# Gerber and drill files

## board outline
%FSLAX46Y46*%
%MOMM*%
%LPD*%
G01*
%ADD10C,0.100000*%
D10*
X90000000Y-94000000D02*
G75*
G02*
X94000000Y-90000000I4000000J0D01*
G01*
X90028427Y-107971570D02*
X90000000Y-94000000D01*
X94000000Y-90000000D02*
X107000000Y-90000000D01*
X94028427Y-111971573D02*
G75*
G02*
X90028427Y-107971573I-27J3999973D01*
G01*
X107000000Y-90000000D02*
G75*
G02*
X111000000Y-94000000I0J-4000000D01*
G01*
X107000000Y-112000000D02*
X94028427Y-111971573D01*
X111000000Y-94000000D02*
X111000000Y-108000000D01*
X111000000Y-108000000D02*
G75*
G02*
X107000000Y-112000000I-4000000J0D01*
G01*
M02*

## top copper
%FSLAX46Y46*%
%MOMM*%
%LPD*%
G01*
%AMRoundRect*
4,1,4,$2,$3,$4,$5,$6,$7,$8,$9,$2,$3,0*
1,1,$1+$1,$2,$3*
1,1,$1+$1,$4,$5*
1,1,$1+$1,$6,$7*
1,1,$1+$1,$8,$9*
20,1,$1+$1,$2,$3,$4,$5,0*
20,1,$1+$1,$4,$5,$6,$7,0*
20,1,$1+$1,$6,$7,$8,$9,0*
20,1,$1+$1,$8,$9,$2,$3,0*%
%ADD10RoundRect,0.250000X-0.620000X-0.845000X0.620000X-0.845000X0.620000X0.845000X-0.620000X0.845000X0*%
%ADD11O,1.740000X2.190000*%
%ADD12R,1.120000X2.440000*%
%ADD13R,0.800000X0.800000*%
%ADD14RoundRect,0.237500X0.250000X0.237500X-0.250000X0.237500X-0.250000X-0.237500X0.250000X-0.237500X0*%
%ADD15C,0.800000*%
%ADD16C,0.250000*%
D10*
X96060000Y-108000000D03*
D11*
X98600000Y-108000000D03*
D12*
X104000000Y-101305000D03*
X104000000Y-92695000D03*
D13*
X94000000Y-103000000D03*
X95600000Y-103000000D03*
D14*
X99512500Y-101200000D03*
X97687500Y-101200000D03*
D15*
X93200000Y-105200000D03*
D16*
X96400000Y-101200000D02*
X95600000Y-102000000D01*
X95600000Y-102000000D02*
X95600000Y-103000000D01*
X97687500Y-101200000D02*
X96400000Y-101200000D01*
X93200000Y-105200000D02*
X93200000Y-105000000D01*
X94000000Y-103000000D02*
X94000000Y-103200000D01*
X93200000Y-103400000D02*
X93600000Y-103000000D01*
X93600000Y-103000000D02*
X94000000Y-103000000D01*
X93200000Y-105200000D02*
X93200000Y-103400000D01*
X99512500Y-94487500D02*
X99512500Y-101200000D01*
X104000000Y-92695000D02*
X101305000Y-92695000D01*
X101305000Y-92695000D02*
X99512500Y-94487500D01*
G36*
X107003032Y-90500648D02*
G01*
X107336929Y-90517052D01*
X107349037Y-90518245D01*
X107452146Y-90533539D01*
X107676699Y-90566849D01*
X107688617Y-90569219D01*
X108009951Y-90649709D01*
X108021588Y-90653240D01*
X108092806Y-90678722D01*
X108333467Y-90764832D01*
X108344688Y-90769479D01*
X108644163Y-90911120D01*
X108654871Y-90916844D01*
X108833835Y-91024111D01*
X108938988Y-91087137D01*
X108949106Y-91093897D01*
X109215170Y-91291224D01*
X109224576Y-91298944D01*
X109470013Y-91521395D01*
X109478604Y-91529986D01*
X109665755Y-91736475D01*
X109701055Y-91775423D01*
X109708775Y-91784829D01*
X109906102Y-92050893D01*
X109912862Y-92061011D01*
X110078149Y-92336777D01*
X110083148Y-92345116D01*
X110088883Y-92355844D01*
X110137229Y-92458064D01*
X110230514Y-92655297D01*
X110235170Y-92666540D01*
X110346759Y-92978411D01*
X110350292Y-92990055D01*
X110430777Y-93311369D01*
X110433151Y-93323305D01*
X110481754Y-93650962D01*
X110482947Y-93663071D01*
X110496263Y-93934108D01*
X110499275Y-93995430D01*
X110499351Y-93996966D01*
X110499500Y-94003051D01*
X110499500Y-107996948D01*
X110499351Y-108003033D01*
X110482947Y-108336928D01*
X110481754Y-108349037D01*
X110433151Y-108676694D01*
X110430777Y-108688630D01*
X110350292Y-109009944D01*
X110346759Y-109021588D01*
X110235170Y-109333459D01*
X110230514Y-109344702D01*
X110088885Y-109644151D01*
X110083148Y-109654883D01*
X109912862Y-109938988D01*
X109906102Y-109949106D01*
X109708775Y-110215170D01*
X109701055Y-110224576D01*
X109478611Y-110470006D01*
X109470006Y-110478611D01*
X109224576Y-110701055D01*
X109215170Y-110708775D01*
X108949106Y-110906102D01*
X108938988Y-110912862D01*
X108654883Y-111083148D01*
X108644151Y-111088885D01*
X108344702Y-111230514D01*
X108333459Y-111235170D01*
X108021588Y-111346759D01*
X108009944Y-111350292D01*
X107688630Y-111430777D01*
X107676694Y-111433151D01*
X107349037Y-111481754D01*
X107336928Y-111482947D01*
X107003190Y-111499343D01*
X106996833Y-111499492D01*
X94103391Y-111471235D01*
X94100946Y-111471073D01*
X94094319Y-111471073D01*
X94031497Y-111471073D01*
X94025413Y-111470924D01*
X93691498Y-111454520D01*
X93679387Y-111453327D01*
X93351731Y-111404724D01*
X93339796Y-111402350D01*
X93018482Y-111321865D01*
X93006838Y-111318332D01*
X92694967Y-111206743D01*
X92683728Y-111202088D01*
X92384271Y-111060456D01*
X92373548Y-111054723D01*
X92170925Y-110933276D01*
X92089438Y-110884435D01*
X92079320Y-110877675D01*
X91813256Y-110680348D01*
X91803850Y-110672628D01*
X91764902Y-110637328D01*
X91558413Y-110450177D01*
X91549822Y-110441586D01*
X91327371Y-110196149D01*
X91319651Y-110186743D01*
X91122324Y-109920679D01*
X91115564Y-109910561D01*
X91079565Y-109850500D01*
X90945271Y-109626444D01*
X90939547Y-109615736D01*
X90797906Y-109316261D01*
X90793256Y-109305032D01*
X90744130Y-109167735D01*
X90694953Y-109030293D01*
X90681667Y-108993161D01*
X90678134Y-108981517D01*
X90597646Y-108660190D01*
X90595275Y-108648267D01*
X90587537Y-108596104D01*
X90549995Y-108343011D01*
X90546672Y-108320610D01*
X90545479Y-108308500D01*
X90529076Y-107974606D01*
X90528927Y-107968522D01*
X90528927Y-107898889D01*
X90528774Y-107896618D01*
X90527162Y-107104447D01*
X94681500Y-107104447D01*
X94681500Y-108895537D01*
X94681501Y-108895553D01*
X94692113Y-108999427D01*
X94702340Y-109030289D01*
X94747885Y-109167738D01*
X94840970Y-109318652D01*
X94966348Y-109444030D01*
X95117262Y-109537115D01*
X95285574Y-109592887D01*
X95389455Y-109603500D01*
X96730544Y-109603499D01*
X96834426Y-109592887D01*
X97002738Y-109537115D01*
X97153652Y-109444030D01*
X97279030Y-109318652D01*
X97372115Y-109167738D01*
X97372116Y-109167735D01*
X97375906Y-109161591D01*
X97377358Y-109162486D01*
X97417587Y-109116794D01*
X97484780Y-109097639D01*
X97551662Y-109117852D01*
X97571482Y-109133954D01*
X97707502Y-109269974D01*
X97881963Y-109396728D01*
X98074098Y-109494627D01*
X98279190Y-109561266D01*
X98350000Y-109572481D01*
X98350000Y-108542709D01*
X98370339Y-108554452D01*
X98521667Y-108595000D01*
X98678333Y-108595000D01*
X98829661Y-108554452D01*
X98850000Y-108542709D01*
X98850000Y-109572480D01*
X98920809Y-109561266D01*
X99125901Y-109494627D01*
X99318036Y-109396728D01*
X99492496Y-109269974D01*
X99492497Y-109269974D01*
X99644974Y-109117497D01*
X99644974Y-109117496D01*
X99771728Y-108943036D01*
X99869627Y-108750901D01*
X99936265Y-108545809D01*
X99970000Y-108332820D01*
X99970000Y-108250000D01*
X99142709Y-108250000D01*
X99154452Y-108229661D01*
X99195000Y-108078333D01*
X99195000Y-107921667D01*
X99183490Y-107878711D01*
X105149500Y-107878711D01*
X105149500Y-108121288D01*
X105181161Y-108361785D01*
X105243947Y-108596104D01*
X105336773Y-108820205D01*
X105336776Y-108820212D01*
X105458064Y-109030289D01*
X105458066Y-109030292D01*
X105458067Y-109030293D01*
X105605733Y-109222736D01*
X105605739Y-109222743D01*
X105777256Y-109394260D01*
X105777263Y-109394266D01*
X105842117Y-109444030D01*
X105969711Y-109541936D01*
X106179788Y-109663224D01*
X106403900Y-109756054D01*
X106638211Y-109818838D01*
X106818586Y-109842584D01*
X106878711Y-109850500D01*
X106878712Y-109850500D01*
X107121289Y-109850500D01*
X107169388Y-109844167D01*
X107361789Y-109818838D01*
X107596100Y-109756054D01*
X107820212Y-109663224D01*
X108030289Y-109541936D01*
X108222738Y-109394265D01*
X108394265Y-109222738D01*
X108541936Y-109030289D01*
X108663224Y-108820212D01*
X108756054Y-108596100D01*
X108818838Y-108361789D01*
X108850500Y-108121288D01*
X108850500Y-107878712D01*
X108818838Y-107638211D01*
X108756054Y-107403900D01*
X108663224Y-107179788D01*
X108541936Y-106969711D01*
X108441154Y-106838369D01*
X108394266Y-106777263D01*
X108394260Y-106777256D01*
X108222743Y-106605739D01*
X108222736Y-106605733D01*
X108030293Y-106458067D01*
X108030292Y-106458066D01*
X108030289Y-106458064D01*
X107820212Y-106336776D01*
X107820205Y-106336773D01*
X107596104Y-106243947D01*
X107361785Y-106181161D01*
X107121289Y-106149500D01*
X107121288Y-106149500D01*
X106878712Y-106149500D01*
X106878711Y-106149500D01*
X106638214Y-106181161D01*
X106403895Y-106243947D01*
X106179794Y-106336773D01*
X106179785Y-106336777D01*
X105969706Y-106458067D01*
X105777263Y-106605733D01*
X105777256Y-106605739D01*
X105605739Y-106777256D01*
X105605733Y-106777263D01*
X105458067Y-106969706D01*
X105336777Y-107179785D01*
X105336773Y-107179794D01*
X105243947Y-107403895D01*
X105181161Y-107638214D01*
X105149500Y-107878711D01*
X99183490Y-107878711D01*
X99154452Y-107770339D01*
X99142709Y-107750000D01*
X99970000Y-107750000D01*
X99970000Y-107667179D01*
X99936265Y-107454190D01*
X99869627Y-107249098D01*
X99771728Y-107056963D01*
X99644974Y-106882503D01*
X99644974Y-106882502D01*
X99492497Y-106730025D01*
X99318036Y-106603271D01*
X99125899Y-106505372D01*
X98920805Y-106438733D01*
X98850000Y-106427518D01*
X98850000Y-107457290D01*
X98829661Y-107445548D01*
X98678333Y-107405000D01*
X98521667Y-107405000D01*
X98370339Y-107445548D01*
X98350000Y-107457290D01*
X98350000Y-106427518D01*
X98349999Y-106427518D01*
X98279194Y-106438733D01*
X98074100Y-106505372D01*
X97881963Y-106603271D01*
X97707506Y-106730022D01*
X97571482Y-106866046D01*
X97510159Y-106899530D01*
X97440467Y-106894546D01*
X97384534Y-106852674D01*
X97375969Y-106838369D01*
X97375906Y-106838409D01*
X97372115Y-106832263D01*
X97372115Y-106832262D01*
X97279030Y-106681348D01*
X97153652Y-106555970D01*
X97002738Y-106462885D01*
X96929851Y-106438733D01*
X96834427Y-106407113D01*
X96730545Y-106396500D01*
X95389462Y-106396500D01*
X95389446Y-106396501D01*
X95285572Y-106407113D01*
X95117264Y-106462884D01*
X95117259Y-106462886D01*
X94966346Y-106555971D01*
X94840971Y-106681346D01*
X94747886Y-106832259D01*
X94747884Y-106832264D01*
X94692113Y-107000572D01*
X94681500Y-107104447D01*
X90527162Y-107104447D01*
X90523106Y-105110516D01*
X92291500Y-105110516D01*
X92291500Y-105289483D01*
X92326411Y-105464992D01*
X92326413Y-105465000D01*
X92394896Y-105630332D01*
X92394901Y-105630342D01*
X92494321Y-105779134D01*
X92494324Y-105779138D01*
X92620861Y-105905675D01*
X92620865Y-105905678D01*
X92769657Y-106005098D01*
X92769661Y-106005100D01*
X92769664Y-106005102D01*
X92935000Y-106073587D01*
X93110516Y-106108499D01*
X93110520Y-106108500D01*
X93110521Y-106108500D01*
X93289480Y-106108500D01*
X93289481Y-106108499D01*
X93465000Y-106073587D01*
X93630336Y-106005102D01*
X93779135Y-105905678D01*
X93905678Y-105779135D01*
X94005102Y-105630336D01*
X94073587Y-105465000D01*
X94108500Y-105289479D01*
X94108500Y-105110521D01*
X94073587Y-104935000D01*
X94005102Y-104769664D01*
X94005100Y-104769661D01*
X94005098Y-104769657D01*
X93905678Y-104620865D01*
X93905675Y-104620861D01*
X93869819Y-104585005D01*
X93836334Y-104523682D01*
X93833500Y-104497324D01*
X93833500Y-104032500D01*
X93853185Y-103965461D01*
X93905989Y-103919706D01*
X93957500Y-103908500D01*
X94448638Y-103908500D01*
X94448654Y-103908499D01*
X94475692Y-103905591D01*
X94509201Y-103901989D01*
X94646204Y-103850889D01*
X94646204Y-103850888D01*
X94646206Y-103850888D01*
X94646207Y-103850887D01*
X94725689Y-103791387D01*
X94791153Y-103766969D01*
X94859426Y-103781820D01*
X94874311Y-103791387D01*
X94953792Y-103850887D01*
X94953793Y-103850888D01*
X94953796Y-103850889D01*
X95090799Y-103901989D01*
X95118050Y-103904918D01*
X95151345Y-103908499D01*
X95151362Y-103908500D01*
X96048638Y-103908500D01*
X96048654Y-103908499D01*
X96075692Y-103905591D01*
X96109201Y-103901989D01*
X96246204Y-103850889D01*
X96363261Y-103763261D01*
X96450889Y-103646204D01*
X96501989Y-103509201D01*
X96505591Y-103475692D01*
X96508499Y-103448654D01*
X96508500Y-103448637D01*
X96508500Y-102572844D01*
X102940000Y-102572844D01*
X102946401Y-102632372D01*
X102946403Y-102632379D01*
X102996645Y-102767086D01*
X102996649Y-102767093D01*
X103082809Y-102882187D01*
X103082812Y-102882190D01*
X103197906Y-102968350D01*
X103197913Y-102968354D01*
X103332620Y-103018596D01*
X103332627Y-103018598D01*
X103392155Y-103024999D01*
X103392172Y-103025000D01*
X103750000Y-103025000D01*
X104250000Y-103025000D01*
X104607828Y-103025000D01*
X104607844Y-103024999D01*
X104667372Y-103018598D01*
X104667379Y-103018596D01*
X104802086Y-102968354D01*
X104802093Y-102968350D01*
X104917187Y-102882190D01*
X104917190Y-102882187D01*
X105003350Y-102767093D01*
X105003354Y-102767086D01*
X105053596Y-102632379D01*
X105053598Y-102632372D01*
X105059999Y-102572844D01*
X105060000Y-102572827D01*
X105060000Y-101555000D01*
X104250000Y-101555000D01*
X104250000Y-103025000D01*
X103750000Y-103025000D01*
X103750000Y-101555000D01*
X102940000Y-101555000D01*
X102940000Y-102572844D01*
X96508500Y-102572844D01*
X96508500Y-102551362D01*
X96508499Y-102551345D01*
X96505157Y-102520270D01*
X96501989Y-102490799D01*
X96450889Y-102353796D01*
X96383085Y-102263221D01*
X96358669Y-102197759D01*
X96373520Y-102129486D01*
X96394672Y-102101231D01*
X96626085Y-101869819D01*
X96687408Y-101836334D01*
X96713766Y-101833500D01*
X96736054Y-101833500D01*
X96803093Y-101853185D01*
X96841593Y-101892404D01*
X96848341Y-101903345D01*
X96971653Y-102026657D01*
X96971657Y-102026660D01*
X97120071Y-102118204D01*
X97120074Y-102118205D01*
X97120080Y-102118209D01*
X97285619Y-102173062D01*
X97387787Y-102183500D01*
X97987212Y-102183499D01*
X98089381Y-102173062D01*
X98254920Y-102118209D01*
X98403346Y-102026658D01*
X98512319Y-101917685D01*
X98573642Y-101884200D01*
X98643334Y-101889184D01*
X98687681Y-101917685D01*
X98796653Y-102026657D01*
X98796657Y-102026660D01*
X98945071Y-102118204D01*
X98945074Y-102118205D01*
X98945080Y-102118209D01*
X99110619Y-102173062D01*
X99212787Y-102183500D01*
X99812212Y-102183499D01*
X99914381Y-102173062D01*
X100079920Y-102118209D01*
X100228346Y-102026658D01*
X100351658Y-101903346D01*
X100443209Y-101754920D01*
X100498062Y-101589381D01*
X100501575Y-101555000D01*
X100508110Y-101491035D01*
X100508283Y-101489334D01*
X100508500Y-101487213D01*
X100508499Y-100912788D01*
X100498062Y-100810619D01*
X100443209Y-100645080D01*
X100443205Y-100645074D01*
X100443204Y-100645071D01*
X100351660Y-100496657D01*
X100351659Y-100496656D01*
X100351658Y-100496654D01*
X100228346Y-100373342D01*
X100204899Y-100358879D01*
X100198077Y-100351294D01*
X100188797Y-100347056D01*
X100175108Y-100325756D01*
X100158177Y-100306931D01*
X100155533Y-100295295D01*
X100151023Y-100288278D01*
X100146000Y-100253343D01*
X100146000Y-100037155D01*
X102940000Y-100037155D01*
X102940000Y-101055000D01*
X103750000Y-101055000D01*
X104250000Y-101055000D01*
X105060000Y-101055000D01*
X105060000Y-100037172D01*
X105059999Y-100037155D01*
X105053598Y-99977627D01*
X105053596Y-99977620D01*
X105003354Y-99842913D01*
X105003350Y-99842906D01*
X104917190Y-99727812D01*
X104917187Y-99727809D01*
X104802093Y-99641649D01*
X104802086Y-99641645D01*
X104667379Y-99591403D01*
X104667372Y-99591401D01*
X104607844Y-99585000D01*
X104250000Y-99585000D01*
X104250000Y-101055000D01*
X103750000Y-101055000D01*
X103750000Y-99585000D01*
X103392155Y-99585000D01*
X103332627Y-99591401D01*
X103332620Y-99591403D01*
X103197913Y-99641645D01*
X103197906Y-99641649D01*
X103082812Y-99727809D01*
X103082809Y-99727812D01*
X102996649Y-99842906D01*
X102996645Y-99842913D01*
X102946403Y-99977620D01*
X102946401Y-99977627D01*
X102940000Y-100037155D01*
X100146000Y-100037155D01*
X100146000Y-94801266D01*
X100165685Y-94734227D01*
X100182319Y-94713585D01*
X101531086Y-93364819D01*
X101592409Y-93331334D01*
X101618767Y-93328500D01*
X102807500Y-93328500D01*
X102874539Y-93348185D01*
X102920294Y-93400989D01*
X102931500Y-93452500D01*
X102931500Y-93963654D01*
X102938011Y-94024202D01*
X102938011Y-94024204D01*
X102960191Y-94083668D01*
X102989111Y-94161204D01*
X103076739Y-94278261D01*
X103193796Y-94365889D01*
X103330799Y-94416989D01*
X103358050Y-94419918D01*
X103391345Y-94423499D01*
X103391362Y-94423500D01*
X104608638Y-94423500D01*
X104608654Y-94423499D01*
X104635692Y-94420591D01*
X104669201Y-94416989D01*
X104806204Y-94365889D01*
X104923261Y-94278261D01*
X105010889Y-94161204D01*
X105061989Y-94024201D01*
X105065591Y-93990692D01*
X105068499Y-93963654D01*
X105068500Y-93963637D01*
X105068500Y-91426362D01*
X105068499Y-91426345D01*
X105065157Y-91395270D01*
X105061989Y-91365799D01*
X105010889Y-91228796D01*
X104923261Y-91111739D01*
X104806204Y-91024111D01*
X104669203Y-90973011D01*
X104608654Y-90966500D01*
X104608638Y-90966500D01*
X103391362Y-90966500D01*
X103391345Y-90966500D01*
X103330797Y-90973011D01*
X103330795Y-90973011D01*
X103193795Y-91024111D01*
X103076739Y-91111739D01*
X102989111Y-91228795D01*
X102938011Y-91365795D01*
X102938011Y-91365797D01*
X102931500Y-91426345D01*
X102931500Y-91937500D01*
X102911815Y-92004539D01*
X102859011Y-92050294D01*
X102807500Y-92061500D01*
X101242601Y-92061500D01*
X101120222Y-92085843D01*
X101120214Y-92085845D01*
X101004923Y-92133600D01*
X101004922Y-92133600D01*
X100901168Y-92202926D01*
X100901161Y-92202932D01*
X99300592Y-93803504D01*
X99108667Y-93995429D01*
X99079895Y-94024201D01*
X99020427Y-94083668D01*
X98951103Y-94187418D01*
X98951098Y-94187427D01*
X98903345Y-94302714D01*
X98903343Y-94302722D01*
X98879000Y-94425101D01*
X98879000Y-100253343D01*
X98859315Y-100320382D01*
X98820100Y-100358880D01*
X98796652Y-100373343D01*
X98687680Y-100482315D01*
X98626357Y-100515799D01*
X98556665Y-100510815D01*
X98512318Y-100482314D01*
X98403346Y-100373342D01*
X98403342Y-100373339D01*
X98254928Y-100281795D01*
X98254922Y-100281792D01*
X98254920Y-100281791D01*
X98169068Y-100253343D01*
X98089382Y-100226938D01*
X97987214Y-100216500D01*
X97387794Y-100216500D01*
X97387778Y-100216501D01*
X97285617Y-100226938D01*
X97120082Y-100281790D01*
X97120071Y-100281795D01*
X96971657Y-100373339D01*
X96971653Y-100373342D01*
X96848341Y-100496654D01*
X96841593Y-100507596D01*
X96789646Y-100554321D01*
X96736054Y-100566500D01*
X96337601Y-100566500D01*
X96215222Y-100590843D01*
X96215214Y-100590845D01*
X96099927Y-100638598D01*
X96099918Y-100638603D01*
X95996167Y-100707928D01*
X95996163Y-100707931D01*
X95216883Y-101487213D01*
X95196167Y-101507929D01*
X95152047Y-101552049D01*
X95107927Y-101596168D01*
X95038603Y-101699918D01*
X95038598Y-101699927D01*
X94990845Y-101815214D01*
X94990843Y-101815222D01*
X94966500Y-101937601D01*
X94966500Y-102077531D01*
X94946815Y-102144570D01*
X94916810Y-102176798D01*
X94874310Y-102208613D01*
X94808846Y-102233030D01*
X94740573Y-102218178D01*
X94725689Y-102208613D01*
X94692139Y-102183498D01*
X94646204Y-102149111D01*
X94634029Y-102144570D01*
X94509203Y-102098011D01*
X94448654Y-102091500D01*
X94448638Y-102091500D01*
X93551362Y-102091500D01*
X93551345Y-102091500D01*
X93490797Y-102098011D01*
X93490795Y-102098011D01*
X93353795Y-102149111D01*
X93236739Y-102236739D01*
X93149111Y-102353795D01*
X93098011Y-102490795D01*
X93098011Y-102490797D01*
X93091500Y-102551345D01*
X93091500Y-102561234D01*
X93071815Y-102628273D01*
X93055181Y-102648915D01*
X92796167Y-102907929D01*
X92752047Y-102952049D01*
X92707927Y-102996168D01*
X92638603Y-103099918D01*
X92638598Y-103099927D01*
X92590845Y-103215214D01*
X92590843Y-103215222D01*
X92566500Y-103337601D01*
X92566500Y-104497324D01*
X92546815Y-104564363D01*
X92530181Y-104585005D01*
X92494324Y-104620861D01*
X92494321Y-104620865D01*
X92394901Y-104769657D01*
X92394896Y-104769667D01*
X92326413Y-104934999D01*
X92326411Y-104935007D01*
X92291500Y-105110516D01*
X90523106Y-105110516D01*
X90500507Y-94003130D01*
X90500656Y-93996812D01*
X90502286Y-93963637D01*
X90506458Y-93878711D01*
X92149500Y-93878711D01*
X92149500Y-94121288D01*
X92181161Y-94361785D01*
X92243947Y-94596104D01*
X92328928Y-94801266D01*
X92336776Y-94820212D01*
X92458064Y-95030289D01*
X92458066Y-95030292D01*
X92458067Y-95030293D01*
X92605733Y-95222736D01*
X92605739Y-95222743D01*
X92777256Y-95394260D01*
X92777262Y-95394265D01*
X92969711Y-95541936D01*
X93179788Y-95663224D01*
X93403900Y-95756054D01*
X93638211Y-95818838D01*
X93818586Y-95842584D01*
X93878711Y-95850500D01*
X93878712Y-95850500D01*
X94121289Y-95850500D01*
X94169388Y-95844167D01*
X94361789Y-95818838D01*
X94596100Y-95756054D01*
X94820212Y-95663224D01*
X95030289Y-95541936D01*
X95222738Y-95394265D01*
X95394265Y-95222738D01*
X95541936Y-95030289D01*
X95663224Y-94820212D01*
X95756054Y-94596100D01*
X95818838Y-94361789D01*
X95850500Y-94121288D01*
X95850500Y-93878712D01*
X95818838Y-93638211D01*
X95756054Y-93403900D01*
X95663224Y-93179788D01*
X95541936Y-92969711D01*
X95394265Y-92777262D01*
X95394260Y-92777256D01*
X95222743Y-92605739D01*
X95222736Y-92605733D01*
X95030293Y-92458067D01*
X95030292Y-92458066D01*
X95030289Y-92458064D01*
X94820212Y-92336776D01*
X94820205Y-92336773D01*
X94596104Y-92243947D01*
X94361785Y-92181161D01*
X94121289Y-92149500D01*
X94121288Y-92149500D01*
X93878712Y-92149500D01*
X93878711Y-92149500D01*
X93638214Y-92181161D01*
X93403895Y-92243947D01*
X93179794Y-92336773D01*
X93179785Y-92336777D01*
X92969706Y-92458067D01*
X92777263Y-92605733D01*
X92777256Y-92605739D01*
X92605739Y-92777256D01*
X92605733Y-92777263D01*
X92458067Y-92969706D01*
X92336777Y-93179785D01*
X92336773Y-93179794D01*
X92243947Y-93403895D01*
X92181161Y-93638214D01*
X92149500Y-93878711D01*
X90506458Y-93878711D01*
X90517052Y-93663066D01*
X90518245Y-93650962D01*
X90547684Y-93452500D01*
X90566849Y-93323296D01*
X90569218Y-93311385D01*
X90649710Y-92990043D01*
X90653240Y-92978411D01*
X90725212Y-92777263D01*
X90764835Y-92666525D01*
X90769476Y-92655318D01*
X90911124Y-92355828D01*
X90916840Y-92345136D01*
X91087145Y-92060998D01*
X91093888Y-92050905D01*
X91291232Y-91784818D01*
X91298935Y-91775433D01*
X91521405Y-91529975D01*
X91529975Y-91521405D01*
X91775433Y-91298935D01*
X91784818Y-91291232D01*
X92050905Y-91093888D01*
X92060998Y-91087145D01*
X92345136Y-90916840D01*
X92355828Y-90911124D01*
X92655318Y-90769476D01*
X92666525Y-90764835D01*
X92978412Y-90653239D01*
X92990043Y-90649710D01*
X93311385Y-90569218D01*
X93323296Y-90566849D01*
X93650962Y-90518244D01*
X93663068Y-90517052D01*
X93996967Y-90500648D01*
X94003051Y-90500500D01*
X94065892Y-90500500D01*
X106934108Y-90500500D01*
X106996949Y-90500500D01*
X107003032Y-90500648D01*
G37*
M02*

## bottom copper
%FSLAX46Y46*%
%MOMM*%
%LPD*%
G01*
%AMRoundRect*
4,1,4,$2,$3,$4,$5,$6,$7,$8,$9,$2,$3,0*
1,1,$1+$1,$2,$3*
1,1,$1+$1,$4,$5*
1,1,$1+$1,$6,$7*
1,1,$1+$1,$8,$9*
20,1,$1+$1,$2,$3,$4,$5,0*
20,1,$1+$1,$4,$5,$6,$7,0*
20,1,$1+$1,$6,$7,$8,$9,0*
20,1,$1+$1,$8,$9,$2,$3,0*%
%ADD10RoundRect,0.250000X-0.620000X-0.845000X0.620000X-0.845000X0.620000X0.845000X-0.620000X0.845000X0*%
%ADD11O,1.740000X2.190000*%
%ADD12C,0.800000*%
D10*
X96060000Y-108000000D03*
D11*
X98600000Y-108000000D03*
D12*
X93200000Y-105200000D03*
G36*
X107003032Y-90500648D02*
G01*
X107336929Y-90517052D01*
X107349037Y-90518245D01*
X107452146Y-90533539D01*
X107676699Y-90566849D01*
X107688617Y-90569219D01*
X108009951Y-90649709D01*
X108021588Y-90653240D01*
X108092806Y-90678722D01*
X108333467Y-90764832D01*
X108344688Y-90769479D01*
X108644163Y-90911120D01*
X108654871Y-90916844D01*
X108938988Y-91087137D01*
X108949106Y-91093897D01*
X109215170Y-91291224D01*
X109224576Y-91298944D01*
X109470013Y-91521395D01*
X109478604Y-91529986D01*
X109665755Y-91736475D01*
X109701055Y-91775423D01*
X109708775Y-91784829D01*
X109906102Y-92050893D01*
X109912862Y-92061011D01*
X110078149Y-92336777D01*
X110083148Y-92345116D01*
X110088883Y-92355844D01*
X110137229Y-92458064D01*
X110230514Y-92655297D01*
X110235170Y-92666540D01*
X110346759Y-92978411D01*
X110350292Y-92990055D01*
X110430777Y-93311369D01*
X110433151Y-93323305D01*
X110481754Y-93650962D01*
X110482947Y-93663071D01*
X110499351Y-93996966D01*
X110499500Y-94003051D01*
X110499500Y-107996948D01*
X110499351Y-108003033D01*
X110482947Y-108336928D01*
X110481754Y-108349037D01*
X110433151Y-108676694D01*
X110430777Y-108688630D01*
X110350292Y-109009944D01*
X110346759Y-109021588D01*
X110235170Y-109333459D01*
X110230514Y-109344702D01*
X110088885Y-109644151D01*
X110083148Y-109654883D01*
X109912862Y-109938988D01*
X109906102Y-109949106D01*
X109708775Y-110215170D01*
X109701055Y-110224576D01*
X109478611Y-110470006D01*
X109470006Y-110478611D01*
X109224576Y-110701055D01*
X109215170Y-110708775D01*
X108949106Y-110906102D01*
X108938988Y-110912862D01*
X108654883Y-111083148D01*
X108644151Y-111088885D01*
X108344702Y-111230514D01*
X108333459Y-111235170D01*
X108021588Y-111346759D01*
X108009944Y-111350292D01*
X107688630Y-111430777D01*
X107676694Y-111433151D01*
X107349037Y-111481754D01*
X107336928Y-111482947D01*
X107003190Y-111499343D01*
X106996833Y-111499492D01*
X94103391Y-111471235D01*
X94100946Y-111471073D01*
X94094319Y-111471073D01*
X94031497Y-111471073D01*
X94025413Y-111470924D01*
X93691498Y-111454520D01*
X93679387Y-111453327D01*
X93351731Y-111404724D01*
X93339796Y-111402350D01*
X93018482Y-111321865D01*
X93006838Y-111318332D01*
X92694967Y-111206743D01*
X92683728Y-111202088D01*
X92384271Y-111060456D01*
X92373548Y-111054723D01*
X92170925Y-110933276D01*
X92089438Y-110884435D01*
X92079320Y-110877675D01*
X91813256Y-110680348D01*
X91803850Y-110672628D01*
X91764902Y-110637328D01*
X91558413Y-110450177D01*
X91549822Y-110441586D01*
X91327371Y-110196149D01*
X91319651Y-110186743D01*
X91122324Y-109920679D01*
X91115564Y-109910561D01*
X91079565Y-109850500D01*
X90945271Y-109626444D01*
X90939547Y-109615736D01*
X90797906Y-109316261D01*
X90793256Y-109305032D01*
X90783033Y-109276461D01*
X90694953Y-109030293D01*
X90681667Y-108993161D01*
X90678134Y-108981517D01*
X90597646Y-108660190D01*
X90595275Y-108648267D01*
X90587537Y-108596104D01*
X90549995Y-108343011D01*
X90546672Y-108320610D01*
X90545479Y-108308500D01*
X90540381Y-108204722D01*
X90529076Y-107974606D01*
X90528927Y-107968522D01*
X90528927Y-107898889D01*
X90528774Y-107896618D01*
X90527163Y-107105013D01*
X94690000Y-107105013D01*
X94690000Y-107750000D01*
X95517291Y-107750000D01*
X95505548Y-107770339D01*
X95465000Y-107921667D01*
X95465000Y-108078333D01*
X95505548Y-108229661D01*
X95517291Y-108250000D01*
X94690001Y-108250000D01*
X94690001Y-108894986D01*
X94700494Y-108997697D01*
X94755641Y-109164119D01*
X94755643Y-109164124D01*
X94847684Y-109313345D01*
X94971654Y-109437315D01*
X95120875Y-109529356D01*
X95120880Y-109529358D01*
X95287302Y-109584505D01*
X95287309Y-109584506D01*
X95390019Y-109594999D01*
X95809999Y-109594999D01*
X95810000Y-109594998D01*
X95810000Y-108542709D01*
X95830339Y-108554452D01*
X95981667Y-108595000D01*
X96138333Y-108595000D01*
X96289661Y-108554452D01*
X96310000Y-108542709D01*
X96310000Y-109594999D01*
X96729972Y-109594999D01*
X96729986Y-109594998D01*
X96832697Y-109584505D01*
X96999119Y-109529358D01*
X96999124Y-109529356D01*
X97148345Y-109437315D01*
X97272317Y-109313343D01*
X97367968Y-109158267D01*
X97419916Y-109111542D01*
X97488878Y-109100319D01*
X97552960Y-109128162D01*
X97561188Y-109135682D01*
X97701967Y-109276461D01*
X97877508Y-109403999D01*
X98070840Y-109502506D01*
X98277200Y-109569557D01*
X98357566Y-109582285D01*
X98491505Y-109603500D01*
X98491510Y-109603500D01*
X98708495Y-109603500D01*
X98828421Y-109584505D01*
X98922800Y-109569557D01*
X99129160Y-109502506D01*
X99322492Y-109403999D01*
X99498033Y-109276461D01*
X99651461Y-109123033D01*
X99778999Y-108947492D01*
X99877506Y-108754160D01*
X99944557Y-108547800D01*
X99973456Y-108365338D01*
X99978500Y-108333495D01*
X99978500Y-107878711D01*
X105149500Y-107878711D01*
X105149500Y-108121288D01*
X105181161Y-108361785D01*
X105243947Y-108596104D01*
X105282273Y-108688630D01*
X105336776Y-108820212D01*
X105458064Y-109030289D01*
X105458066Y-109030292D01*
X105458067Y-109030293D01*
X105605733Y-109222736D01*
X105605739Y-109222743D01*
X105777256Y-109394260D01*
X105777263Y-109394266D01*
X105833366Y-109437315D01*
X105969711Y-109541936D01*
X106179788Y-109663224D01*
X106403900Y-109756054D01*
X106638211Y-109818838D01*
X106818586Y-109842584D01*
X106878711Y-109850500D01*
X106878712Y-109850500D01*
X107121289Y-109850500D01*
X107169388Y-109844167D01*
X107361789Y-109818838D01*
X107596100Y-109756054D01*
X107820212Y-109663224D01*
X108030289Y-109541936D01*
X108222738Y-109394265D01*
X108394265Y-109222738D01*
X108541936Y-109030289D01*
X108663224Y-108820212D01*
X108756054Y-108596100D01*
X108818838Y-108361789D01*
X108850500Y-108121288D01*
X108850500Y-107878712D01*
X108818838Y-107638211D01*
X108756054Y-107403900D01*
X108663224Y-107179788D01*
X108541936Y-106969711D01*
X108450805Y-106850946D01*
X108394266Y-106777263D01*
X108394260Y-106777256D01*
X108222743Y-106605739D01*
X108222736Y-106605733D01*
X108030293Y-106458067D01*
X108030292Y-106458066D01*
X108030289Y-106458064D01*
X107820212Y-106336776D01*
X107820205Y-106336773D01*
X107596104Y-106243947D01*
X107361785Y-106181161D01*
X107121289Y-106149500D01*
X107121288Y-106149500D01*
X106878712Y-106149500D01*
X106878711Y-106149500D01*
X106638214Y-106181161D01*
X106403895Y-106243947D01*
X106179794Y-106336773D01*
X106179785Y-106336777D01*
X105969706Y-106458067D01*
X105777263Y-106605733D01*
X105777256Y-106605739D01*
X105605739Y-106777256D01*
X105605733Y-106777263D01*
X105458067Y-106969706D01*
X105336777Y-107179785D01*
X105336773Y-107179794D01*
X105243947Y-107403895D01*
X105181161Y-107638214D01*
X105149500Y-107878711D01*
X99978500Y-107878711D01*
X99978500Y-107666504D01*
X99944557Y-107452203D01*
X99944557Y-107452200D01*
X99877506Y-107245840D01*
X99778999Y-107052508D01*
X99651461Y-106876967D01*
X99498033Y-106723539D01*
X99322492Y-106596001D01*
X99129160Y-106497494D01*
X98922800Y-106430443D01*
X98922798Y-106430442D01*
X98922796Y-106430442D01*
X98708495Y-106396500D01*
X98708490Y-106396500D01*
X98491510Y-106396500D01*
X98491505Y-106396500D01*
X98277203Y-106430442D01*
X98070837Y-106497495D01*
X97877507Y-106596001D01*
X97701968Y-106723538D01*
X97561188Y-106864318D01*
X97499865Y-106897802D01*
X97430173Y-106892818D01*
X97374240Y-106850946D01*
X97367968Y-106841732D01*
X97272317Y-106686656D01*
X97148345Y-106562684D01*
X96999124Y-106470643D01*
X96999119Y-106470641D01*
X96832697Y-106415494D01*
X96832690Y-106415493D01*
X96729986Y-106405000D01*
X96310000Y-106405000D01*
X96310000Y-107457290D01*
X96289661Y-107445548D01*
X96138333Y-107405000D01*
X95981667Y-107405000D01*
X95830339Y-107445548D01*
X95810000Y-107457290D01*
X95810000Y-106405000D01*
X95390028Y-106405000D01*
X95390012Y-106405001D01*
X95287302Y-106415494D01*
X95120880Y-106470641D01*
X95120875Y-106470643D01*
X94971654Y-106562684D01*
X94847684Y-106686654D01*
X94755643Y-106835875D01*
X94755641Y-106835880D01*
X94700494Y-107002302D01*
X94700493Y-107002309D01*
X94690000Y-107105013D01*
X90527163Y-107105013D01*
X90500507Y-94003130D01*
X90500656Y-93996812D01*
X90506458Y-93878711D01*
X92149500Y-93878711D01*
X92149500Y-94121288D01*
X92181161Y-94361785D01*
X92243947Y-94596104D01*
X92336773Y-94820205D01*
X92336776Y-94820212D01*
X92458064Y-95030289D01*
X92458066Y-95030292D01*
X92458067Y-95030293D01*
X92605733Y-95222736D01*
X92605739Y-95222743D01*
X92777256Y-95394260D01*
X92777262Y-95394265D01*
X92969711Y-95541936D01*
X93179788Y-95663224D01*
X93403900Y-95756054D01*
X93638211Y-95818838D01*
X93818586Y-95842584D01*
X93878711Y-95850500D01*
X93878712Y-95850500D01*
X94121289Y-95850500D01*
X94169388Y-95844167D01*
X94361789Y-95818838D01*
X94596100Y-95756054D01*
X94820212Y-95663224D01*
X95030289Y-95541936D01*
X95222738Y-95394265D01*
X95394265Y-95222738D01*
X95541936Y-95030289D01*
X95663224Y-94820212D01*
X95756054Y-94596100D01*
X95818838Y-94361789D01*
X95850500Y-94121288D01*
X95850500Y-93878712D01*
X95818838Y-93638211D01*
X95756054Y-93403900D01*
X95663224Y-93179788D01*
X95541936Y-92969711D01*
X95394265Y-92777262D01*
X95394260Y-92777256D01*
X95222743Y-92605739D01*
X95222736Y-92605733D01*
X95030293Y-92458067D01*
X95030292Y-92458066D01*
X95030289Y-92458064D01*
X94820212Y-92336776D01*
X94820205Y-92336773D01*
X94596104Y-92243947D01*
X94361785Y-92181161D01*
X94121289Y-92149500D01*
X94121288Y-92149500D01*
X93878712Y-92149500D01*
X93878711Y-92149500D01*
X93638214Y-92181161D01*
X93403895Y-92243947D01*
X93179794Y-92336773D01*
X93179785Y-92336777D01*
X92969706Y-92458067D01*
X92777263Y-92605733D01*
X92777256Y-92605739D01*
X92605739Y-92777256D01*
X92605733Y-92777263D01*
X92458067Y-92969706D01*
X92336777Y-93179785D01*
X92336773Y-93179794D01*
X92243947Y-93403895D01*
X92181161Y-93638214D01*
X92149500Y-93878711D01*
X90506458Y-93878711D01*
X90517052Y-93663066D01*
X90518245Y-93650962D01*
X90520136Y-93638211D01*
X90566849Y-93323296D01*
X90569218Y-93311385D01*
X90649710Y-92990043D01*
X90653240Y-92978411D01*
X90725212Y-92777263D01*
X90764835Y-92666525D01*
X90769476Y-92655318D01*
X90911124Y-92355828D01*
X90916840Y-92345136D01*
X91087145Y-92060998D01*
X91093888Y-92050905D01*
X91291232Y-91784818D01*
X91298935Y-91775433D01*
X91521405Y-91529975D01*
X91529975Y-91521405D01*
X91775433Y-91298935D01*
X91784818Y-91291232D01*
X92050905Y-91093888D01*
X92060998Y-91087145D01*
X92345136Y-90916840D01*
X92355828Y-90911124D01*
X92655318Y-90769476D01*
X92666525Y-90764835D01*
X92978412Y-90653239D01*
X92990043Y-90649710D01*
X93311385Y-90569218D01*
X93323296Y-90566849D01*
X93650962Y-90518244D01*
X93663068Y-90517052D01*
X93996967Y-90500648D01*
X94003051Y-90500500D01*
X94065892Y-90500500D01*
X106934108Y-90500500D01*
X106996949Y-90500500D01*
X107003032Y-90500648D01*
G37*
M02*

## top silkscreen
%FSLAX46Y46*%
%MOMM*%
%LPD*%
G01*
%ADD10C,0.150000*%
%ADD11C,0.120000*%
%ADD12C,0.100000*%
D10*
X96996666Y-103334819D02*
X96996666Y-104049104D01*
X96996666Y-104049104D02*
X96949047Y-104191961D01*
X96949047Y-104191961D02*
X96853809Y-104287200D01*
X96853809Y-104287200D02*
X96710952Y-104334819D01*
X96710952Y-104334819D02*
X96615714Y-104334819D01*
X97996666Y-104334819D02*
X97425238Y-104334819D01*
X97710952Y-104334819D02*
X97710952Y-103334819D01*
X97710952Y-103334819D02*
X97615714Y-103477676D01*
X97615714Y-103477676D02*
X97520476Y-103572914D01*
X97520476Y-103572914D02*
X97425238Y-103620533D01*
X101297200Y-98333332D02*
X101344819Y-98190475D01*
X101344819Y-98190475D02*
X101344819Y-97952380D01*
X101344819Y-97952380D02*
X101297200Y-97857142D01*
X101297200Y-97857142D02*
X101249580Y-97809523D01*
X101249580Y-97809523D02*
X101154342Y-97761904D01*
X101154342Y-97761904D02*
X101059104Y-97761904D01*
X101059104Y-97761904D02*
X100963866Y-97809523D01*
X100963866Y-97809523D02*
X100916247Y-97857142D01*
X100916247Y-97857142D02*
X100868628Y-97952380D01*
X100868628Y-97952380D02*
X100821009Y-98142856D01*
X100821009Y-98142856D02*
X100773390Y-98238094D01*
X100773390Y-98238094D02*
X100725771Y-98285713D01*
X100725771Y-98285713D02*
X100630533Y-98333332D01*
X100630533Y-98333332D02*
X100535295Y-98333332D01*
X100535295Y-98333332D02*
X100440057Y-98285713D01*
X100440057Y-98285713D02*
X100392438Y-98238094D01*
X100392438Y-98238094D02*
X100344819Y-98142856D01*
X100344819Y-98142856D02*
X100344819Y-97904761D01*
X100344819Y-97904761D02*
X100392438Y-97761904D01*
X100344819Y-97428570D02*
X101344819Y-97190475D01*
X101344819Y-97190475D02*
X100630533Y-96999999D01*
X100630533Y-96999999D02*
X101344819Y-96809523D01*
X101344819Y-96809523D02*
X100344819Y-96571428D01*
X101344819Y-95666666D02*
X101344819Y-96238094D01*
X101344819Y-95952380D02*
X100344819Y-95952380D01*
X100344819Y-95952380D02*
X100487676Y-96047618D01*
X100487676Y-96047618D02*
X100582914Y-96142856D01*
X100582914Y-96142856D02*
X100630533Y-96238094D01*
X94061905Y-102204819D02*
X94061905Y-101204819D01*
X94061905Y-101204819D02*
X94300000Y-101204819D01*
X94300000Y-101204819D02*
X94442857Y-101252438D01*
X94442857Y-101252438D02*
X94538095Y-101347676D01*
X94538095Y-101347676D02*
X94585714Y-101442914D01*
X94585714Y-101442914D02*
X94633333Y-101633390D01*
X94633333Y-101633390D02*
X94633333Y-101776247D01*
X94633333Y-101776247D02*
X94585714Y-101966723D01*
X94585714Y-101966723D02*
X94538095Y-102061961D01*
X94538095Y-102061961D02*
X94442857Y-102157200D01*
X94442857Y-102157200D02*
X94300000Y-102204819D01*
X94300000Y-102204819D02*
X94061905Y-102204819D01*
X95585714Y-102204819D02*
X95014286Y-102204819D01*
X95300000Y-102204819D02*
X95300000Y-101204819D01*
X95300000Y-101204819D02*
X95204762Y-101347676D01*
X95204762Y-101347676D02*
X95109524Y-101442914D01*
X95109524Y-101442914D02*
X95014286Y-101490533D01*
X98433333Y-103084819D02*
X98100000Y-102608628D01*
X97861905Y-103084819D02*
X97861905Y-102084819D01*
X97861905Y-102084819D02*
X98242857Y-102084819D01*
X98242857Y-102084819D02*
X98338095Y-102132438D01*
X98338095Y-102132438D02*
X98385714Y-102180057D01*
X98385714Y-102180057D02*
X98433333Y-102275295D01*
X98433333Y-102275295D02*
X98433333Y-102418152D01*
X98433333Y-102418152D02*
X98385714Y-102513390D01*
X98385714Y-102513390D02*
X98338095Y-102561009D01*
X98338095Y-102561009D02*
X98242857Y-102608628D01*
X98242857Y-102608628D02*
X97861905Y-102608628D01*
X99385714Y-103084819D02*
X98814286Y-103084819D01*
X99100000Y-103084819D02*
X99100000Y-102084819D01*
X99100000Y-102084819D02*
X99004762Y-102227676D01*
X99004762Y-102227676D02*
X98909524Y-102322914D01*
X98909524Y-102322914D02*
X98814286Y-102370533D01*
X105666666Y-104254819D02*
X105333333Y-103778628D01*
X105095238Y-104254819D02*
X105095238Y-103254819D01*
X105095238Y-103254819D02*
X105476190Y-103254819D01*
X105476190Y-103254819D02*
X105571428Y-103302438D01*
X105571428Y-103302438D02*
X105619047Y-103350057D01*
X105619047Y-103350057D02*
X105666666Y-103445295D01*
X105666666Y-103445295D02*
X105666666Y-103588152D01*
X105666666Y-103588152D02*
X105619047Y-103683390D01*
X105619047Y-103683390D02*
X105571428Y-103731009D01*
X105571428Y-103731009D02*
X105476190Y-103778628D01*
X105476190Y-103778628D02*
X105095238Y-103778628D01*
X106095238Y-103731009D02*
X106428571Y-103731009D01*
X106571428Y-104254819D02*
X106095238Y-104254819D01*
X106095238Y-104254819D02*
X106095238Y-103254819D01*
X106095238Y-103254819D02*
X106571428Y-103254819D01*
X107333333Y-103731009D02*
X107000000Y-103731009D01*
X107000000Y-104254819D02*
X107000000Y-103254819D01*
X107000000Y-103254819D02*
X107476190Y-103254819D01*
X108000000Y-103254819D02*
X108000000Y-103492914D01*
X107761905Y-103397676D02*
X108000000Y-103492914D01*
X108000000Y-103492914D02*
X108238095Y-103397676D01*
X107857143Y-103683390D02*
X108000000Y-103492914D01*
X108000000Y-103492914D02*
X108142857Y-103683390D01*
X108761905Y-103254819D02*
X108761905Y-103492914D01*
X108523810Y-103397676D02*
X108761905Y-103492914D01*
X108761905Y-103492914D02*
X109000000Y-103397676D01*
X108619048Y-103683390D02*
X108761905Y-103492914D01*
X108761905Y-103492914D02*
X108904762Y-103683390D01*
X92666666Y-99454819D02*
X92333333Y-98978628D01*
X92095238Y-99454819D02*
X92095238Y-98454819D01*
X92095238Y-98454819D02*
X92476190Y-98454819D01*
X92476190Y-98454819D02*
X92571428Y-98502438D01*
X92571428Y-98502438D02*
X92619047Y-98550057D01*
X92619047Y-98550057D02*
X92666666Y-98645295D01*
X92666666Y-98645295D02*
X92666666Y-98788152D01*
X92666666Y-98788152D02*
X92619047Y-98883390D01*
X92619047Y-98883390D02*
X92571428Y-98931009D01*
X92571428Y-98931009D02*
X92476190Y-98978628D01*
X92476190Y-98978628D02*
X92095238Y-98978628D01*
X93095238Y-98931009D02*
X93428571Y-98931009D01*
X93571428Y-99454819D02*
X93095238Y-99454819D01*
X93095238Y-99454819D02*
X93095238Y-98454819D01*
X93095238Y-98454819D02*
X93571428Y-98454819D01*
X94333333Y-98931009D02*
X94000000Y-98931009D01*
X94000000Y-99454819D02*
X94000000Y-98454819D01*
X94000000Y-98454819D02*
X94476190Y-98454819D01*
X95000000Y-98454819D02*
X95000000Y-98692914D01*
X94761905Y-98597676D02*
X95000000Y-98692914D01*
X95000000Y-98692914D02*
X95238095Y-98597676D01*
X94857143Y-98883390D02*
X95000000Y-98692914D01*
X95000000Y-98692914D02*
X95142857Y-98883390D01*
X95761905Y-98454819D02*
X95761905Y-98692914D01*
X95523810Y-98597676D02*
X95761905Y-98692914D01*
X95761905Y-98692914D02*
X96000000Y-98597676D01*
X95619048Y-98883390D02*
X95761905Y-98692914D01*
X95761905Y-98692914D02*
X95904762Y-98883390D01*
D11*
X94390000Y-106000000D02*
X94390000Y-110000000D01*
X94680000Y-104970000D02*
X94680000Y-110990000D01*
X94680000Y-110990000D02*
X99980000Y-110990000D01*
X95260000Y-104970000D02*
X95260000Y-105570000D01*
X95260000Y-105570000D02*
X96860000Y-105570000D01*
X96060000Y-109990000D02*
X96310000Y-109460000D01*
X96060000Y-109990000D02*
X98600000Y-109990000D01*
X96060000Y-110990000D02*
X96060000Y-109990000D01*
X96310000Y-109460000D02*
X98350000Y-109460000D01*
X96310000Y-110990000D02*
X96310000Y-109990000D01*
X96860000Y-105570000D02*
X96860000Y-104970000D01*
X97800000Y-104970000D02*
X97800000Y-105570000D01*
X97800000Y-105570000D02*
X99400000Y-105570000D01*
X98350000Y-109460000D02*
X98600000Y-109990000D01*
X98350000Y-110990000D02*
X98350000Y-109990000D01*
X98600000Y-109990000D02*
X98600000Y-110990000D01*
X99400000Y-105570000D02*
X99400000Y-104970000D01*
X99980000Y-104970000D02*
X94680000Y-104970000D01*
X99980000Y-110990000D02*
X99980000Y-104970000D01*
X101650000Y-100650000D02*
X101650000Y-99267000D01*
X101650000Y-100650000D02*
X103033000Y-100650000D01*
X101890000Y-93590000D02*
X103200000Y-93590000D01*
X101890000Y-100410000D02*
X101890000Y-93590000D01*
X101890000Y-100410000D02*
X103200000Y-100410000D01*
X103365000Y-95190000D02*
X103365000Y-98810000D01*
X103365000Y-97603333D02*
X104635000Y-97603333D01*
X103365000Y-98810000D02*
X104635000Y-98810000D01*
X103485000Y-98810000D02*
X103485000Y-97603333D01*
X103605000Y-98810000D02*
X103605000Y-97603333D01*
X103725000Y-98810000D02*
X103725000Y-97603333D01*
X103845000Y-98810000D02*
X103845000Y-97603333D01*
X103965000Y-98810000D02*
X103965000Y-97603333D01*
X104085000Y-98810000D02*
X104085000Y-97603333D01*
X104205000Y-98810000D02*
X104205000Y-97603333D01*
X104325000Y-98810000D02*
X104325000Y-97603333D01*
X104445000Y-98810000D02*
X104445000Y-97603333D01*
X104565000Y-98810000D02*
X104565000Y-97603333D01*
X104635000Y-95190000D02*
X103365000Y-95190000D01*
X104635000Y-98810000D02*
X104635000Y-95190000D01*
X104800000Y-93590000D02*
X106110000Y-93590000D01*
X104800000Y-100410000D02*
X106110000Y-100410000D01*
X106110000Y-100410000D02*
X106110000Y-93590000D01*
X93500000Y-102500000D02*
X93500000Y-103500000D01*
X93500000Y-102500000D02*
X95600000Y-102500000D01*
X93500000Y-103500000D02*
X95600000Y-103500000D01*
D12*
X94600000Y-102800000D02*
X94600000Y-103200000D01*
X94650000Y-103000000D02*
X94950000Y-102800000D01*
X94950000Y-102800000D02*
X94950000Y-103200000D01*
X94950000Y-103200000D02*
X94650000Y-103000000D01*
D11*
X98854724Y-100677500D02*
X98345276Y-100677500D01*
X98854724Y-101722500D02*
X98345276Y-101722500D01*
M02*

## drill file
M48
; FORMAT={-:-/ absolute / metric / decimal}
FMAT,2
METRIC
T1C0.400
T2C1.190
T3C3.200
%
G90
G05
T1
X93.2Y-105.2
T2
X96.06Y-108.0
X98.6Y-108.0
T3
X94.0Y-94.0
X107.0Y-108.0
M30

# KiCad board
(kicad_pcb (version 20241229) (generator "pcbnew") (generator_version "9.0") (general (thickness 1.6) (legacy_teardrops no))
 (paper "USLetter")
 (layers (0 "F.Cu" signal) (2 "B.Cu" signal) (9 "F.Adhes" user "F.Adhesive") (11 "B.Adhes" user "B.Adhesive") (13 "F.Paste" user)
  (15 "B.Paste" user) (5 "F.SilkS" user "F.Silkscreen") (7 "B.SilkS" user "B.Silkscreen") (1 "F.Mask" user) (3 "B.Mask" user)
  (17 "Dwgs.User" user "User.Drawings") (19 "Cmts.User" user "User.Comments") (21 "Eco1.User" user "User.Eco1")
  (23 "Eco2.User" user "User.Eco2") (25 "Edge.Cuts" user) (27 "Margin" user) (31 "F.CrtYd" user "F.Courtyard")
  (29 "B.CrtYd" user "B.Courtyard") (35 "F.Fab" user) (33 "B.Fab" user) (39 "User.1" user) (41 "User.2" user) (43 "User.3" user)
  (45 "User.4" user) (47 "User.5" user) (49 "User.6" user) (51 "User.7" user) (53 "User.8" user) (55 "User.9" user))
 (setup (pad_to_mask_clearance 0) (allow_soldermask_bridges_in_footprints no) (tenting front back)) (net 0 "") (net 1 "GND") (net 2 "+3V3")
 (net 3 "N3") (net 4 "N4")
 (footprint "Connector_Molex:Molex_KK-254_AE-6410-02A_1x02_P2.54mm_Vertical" (layer "F.Cu") (at 96.06 108)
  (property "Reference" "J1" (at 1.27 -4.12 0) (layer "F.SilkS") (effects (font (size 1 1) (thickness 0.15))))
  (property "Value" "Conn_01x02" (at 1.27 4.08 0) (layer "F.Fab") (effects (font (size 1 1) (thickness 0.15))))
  (fp_line (start -1.67 -2) (end -1.67 2) (stroke (width 0.12) (type solid)) (layer "F.SilkS"))
  (fp_line (start -1.38 -3.03) (end -1.38 2.99) (stroke (width 0.12) (type solid)) (layer "F.SilkS"))
  (fp_line (start -1.38 2.99) (end 3.92 2.99) (stroke (width 0.12) (type solid)) (layer "F.SilkS"))
  (fp_line (start -0.8 -3.03) (end -0.8 -2.43) (stroke (width 0.12) (type solid)) (layer "F.SilkS"))
  (fp_line (start -0.8 -2.43) (end 0.8 -2.43) (stroke (width 0.12) (type solid)) (layer "F.SilkS"))
  (fp_line (start 0 1.99) (end 0.25 1.46) (stroke (width 0.12) (type solid)) (layer "F.SilkS"))
  (fp_line (start 0 1.99) (end 2.54 1.99) (stroke (width 0.12) (type solid)) (layer "F.SilkS"))
  (fp_line (start 0 2.99) (end 0 1.99) (stroke (width 0.12) (type solid)) (layer "F.SilkS"))
  (fp_line (start 0.25 1.46) (end 2.29 1.46) (stroke (width 0.12) (type solid)) (layer "F.SilkS"))
  (fp_line (start 0.25 2.99) (end 0.25 1.99) (stroke (width 0.12) (type solid)) (layer "F.SilkS"))
  (fp_line (start 0.8 -2.43) (end 0.8 -3.03) (stroke (width 0.12) (type solid)) (layer "F.SilkS"))
  (fp_line (start 1.74 -3.03) (end 1.74 -2.43) (stroke (width 0.12) (type solid)) (layer "F.SilkS"))
  (fp_line (start 1.74 -2.43) (end 3.34 -2.43) (stroke (width 0.12) (type solid)) (layer "F.SilkS"))
  (fp_line (start 2.29 1.46) (end 2.54 1.99) (stroke (width 0.12) (type solid)) (layer "F.SilkS"))
  (fp_line (start 2.29 2.99) (end 2.29 1.99) (stroke (width 0.12) (type solid)) (layer "F.SilkS"))
  (fp_line (start 2.54 1.99) (end 2.54 2.99) (stroke (width 0.12) (type solid)) (layer "F.SilkS"))
  (fp_line (start 3.34 -2.43) (end 3.34 -3.03) (stroke (width 0.12) (type solid)) (layer "F.SilkS"))
  (fp_line (start 3.92 -3.03) (end -1.38 -3.03) (stroke (width 0.12) (type solid)) (layer "F.SilkS"))
  (fp_line (start 3.92 2.99) (end 3.92 -3.03) (stroke (width 0.12) (type solid)) (layer "F.SilkS"))
  (pad "1" thru_hole roundrect (at 0 0) (size 1.74 2.19) (drill 1.19) (layers "*.Cu" "*.Mask") (remove_unused_layers no)
   (roundrect_rratio 0.143678) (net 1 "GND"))
  (pad "2" thru_hole oval (at 2.54 0) (size 1.74 2.19) (drill 1.19) (layers "*.Cu" "*.Mask") (remove_unused_layers no) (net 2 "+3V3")))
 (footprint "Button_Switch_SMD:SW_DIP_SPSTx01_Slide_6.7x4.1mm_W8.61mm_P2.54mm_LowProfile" (layer "F.Cu") (at 104 97 90)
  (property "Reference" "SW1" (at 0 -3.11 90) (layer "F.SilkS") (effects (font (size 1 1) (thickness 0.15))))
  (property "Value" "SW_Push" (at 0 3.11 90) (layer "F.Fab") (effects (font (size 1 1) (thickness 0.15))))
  (fp_line (start -3.65 -2.35) (end -2.267 -2.35) (stroke (width 0.12) (type solid)) (layer "F.SilkS"))
  (fp_line (start -3.65 -2.35) (end -3.65 -0.967) (stroke (width 0.12) (type solid)) (layer "F.SilkS"))
  (fp_line (start 3.41 -2.11) (end 3.41 -0.8) (stroke (width 0.12) (type solid)) (layer "F.SilkS"))
  (fp_line (start -3.41 -2.11) (end 3.41 -2.11) (stroke (width 0.12) (type solid)) (layer "F.SilkS"))
  (fp_line (start -3.41 -2.11) (end -3.41 -0.8) (stroke (width 0.12) (type solid)) (layer "F.SilkS"))
  (fp_line (start 1.81 -0.635) (end -1.81 -0.635) (stroke (width 0.12) (type solid)) (layer "F.SilkS"))
  (fp_line (start -0.603333 -0.635) (end -0.603333 0.635) (stroke (width 0.12) (type solid)) (layer "F.SilkS"))
  (fp_line (start -1.81 -0.635) (end -1.81 0.635) (stroke (width 0.12) (type solid)) (layer "F.SilkS"))
  (fp_line (start -1.81 -0.515) (end -0.603333 -0.515) (stroke (width 0.12) (type solid)) (layer "F.SilkS"))
  (fp_line (start -1.81 -0.395) (end -0.603333 -0.395) (stroke (width 0.12) (type solid)) (layer "F.SilkS"))
  (fp_line (start -1.81 -0.275) (end -0.603333 -0.275) (stroke (width 0.12) (type solid)) (layer "F.SilkS"))
  (fp_line (start -1.81 -0.155) (end -0.603333 -0.155) (stroke (width 0.12) (type solid)) (layer "F.SilkS"))
  (fp_line (start -1.81 -0.035) (end -0.603333 -0.035) (stroke (width 0.12) (type solid)) (layer "F.SilkS"))
  (fp_line (start -1.81 0.085) (end -0.603333 0.085) (stroke (width 0.12) (type solid)) (layer "F.SilkS"))
  (fp_line (start -1.81 0.205) (end -0.603333 0.205) (stroke (width 0.12) (type solid)) (layer "F.SilkS"))
  (fp_line (start -1.81 0.325) (end -0.603333 0.325) (stroke (width 0.12) (type solid)) (layer "F.SilkS"))
  (fp_line (start -1.81 0.445) (end -0.603333 0.445) (stroke (width 0.12) (type solid)) (layer "F.SilkS"))
  (fp_line (start -1.81 0.565) (end -0.603333 0.565) (stroke (width 0.12) (type solid)) (layer "F.SilkS"))
  (fp_line (start 1.81 0.635) (end 1.81 -0.635) (stroke (width 0.12) (type solid)) (layer "F.SilkS"))
  (fp_line (start -1.81 0.635) (end 1.81 0.635) (stroke (width 0.12) (type solid)) (layer "F.SilkS"))
  (fp_line (start 3.41 0.8) (end 3.41 2.11) (stroke (width 0.12) (type solid)) (layer "F.SilkS"))
  (fp_line (start -3.41 0.8) (end -3.41 2.11) (stroke (width 0.12) (type solid)) (layer "F.SilkS"))
  (fp_line (start -3.41 2.11) (end 3.41 2.11) (stroke (width 0.12) (type solid)) (layer "F.SilkS"))
  (pad "1" smd rect (at -4.305 0 90) (size 2.44 1.12) (layers "F.Cu" "F.Mask" "F.Paste") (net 2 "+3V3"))
  (pad "2" smd rect (at 4.305 0 90) (size 2.44 1.12) (layers "F.Cu" "F.Mask" "F.Paste") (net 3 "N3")))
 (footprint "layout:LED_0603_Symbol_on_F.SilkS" (layer "F.Cu") (at 94.8 103)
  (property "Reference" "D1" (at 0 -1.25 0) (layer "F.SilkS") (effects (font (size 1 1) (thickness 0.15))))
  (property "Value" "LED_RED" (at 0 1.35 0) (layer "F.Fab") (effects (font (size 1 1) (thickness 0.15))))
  (fp_line (start -1.3 -0.5) (end -1.3 0.5) (stroke (width 0.12) (type solid)) (layer "F.SilkS"))
  (fp_line (start -1.3 -0.5) (end 0.8 -0.5) (stroke (width 0.12) (type solid)) (layer "F.SilkS"))
  (fp_line (start -1.3 0.5) (end 0.8 0.5) (stroke (width 0.12) (type solid)) (layer "F.SilkS"))
  (fp_line (start -0.2 -0.2) (end -0.2 0.2) (stroke (width 0.1) (type solid)) (layer "F.SilkS"))
  (fp_line (start -0.15 0) (end 0.15 -0.2) (stroke (width 0.1) (type solid)) (layer "F.SilkS"))
  (fp_line (start 0.15 -0.2) (end 0.15 0.2) (stroke (width 0.1) (type solid)) (layer "F.SilkS"))
  (fp_line (start 0.15 0.2) (end -0.15 0) (stroke (width 0.1) (type solid)) (layer "F.SilkS"))
  (pad "1" smd rect (at -0.8 0 180) (size 0.8 0.8) (layers "F.Cu" "F.Mask" "F.Paste") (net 1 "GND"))
  (pad "2" smd rect (at 0.8 0 180) (size 0.8 0.8) (layers "F.Cu" "F.Mask" "F.Paste") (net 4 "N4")))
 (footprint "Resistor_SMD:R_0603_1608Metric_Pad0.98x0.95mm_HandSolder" (layer "F.Cu") (at 98.6 101.2 180)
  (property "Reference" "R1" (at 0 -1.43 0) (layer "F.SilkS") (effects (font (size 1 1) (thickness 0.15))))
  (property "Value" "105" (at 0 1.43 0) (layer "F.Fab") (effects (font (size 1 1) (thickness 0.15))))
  (fp_line (start -0.254724 0.5225) (end 0.254724 0.5225) (stroke (width 0.12) (type solid)) (layer "F.SilkS"))
  (fp_line (start -0.254724 -0.5225) (end 0.254724 -0.5225) (stroke (width 0.12) (type solid)) (layer "F.SilkS"))
  (pad "1" smd roundrect (at -0.9125 0 180) (size 0.975 0.95) (layers "F.Cu" "F.Mask" "F.Paste") (roundrect_rratio 0.25) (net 3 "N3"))
  (pad "2" smd roundrect (at 0.9125 0 180) (size 0.975 0.95) (layers "F.Cu" "F.Mask" "F.Paste") (roundrect_rratio 0.25) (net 4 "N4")))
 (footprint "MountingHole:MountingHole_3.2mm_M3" (layer "F.Cu") (at 107 108)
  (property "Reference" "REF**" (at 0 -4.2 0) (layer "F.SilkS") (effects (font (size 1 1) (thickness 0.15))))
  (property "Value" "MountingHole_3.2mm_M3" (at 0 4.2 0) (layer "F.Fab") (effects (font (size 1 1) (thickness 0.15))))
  (pad "" np_thru_hole circle (at 0 0) (size 3.2 3.2) (drill 3.2) (layers "*.Cu" "*.Mask")))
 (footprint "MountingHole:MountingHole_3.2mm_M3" (layer "F.Cu") (at 94 94)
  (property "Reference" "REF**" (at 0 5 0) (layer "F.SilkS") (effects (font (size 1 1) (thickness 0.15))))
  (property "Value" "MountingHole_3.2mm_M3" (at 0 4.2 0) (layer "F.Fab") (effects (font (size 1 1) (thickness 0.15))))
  (pad "" np_thru_hole circle (at 0 0) (size 3.2 3.2) (drill 3.2) (layers "*.Cu" "*.Mask")))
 (gr_arc (start 90 94) (mid 91.171573 91.171573) (end 94 90) (stroke (width 0.1) (type default)) (layer "Edge.Cuts"))
 (gr_line (start 90.028427 107.97157) (end 90 94) (stroke (width 0.1) (type default)) (layer "Edge.Cuts"))
 (gr_line (start 94 90) (end 107 90) (stroke (width 0.1) (type default)) (layer "Edge.Cuts"))
 (gr_arc (start 94.028427 111.971573) (mid 91.2 110.8) (end 90.028427 107.971573) (stroke (width 0.1) (type default)) (layer "Edge.Cuts"))
 (gr_arc (start 107 90) (mid 109.828427 91.171573) (end 111 94) (stroke (width 0.1) (type default)) (layer "Edge.Cuts"))
 (gr_line (start 107 112) (end 94.028427 111.971573) (stroke (width 0.1) (type default)) (layer "Edge.Cuts"))
 (gr_line (start 111 94) (end 111 108) (stroke (width 0.1) (type default)) (layer "Edge.Cuts"))
 (gr_arc (start 111 108) (mid 109.828427 110.828427) (end 107 112) (stroke (width 0.1) (type default)) (layer "Edge.Cuts"))
 (segment (start 96.4 101.2) (end 95.6 102) (width 0.25) (layer "F.Cu") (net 4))
 (segment (start 95.6 102) (end 95.6 103) (width 0.25) (layer "F.Cu") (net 4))
 (segment (start 97.6875 101.2) (end 96.4 101.2) (width 0.25) (layer "F.Cu") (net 4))
 (segment (start 93.2 105.2) (end 93.2 105) (width 0.25) (layer "F.Cu") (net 1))
 (segment (start 94 103) (end 94 103.2) (width 0.25) (layer "F.Cu") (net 1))
 (segment (start 93.2 103.4) (end 93.6 103) (width 0.25) (layer "F.Cu") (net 1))
 (segment (start 93.6 103) (end 94 103) (width 0.25) (layer "F.Cu") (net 1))
 (segment (start 93.2 105.2) (end 93.2 103.4) (width 0.25) (layer "F.Cu") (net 1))
 (via (at 93.2 105.2) (size 0.8) (drill 0.4) (layers "F.Cu" "B.Cu") (free yes) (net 1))
 (segment (start 99.5125 94.4875) (end 99.5125 101.2) (width 0.25) (layer "F.Cu") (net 3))
 (segment (start 104 92.695) (end 101.305 92.695) (width 0.25) (layer "F.Cu") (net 3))
 (segment (start 101.305 92.695) (end 99.5125 94.4875) (width 0.25) (layer "F.Cu") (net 3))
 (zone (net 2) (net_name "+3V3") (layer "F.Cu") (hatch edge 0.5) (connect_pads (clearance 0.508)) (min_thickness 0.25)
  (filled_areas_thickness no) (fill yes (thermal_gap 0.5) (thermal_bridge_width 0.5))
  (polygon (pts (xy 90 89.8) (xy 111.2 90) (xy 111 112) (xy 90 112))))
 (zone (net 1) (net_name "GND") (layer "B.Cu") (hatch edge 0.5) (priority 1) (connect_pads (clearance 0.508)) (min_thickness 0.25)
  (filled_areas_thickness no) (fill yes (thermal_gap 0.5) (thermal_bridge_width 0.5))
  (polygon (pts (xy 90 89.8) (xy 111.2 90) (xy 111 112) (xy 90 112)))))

